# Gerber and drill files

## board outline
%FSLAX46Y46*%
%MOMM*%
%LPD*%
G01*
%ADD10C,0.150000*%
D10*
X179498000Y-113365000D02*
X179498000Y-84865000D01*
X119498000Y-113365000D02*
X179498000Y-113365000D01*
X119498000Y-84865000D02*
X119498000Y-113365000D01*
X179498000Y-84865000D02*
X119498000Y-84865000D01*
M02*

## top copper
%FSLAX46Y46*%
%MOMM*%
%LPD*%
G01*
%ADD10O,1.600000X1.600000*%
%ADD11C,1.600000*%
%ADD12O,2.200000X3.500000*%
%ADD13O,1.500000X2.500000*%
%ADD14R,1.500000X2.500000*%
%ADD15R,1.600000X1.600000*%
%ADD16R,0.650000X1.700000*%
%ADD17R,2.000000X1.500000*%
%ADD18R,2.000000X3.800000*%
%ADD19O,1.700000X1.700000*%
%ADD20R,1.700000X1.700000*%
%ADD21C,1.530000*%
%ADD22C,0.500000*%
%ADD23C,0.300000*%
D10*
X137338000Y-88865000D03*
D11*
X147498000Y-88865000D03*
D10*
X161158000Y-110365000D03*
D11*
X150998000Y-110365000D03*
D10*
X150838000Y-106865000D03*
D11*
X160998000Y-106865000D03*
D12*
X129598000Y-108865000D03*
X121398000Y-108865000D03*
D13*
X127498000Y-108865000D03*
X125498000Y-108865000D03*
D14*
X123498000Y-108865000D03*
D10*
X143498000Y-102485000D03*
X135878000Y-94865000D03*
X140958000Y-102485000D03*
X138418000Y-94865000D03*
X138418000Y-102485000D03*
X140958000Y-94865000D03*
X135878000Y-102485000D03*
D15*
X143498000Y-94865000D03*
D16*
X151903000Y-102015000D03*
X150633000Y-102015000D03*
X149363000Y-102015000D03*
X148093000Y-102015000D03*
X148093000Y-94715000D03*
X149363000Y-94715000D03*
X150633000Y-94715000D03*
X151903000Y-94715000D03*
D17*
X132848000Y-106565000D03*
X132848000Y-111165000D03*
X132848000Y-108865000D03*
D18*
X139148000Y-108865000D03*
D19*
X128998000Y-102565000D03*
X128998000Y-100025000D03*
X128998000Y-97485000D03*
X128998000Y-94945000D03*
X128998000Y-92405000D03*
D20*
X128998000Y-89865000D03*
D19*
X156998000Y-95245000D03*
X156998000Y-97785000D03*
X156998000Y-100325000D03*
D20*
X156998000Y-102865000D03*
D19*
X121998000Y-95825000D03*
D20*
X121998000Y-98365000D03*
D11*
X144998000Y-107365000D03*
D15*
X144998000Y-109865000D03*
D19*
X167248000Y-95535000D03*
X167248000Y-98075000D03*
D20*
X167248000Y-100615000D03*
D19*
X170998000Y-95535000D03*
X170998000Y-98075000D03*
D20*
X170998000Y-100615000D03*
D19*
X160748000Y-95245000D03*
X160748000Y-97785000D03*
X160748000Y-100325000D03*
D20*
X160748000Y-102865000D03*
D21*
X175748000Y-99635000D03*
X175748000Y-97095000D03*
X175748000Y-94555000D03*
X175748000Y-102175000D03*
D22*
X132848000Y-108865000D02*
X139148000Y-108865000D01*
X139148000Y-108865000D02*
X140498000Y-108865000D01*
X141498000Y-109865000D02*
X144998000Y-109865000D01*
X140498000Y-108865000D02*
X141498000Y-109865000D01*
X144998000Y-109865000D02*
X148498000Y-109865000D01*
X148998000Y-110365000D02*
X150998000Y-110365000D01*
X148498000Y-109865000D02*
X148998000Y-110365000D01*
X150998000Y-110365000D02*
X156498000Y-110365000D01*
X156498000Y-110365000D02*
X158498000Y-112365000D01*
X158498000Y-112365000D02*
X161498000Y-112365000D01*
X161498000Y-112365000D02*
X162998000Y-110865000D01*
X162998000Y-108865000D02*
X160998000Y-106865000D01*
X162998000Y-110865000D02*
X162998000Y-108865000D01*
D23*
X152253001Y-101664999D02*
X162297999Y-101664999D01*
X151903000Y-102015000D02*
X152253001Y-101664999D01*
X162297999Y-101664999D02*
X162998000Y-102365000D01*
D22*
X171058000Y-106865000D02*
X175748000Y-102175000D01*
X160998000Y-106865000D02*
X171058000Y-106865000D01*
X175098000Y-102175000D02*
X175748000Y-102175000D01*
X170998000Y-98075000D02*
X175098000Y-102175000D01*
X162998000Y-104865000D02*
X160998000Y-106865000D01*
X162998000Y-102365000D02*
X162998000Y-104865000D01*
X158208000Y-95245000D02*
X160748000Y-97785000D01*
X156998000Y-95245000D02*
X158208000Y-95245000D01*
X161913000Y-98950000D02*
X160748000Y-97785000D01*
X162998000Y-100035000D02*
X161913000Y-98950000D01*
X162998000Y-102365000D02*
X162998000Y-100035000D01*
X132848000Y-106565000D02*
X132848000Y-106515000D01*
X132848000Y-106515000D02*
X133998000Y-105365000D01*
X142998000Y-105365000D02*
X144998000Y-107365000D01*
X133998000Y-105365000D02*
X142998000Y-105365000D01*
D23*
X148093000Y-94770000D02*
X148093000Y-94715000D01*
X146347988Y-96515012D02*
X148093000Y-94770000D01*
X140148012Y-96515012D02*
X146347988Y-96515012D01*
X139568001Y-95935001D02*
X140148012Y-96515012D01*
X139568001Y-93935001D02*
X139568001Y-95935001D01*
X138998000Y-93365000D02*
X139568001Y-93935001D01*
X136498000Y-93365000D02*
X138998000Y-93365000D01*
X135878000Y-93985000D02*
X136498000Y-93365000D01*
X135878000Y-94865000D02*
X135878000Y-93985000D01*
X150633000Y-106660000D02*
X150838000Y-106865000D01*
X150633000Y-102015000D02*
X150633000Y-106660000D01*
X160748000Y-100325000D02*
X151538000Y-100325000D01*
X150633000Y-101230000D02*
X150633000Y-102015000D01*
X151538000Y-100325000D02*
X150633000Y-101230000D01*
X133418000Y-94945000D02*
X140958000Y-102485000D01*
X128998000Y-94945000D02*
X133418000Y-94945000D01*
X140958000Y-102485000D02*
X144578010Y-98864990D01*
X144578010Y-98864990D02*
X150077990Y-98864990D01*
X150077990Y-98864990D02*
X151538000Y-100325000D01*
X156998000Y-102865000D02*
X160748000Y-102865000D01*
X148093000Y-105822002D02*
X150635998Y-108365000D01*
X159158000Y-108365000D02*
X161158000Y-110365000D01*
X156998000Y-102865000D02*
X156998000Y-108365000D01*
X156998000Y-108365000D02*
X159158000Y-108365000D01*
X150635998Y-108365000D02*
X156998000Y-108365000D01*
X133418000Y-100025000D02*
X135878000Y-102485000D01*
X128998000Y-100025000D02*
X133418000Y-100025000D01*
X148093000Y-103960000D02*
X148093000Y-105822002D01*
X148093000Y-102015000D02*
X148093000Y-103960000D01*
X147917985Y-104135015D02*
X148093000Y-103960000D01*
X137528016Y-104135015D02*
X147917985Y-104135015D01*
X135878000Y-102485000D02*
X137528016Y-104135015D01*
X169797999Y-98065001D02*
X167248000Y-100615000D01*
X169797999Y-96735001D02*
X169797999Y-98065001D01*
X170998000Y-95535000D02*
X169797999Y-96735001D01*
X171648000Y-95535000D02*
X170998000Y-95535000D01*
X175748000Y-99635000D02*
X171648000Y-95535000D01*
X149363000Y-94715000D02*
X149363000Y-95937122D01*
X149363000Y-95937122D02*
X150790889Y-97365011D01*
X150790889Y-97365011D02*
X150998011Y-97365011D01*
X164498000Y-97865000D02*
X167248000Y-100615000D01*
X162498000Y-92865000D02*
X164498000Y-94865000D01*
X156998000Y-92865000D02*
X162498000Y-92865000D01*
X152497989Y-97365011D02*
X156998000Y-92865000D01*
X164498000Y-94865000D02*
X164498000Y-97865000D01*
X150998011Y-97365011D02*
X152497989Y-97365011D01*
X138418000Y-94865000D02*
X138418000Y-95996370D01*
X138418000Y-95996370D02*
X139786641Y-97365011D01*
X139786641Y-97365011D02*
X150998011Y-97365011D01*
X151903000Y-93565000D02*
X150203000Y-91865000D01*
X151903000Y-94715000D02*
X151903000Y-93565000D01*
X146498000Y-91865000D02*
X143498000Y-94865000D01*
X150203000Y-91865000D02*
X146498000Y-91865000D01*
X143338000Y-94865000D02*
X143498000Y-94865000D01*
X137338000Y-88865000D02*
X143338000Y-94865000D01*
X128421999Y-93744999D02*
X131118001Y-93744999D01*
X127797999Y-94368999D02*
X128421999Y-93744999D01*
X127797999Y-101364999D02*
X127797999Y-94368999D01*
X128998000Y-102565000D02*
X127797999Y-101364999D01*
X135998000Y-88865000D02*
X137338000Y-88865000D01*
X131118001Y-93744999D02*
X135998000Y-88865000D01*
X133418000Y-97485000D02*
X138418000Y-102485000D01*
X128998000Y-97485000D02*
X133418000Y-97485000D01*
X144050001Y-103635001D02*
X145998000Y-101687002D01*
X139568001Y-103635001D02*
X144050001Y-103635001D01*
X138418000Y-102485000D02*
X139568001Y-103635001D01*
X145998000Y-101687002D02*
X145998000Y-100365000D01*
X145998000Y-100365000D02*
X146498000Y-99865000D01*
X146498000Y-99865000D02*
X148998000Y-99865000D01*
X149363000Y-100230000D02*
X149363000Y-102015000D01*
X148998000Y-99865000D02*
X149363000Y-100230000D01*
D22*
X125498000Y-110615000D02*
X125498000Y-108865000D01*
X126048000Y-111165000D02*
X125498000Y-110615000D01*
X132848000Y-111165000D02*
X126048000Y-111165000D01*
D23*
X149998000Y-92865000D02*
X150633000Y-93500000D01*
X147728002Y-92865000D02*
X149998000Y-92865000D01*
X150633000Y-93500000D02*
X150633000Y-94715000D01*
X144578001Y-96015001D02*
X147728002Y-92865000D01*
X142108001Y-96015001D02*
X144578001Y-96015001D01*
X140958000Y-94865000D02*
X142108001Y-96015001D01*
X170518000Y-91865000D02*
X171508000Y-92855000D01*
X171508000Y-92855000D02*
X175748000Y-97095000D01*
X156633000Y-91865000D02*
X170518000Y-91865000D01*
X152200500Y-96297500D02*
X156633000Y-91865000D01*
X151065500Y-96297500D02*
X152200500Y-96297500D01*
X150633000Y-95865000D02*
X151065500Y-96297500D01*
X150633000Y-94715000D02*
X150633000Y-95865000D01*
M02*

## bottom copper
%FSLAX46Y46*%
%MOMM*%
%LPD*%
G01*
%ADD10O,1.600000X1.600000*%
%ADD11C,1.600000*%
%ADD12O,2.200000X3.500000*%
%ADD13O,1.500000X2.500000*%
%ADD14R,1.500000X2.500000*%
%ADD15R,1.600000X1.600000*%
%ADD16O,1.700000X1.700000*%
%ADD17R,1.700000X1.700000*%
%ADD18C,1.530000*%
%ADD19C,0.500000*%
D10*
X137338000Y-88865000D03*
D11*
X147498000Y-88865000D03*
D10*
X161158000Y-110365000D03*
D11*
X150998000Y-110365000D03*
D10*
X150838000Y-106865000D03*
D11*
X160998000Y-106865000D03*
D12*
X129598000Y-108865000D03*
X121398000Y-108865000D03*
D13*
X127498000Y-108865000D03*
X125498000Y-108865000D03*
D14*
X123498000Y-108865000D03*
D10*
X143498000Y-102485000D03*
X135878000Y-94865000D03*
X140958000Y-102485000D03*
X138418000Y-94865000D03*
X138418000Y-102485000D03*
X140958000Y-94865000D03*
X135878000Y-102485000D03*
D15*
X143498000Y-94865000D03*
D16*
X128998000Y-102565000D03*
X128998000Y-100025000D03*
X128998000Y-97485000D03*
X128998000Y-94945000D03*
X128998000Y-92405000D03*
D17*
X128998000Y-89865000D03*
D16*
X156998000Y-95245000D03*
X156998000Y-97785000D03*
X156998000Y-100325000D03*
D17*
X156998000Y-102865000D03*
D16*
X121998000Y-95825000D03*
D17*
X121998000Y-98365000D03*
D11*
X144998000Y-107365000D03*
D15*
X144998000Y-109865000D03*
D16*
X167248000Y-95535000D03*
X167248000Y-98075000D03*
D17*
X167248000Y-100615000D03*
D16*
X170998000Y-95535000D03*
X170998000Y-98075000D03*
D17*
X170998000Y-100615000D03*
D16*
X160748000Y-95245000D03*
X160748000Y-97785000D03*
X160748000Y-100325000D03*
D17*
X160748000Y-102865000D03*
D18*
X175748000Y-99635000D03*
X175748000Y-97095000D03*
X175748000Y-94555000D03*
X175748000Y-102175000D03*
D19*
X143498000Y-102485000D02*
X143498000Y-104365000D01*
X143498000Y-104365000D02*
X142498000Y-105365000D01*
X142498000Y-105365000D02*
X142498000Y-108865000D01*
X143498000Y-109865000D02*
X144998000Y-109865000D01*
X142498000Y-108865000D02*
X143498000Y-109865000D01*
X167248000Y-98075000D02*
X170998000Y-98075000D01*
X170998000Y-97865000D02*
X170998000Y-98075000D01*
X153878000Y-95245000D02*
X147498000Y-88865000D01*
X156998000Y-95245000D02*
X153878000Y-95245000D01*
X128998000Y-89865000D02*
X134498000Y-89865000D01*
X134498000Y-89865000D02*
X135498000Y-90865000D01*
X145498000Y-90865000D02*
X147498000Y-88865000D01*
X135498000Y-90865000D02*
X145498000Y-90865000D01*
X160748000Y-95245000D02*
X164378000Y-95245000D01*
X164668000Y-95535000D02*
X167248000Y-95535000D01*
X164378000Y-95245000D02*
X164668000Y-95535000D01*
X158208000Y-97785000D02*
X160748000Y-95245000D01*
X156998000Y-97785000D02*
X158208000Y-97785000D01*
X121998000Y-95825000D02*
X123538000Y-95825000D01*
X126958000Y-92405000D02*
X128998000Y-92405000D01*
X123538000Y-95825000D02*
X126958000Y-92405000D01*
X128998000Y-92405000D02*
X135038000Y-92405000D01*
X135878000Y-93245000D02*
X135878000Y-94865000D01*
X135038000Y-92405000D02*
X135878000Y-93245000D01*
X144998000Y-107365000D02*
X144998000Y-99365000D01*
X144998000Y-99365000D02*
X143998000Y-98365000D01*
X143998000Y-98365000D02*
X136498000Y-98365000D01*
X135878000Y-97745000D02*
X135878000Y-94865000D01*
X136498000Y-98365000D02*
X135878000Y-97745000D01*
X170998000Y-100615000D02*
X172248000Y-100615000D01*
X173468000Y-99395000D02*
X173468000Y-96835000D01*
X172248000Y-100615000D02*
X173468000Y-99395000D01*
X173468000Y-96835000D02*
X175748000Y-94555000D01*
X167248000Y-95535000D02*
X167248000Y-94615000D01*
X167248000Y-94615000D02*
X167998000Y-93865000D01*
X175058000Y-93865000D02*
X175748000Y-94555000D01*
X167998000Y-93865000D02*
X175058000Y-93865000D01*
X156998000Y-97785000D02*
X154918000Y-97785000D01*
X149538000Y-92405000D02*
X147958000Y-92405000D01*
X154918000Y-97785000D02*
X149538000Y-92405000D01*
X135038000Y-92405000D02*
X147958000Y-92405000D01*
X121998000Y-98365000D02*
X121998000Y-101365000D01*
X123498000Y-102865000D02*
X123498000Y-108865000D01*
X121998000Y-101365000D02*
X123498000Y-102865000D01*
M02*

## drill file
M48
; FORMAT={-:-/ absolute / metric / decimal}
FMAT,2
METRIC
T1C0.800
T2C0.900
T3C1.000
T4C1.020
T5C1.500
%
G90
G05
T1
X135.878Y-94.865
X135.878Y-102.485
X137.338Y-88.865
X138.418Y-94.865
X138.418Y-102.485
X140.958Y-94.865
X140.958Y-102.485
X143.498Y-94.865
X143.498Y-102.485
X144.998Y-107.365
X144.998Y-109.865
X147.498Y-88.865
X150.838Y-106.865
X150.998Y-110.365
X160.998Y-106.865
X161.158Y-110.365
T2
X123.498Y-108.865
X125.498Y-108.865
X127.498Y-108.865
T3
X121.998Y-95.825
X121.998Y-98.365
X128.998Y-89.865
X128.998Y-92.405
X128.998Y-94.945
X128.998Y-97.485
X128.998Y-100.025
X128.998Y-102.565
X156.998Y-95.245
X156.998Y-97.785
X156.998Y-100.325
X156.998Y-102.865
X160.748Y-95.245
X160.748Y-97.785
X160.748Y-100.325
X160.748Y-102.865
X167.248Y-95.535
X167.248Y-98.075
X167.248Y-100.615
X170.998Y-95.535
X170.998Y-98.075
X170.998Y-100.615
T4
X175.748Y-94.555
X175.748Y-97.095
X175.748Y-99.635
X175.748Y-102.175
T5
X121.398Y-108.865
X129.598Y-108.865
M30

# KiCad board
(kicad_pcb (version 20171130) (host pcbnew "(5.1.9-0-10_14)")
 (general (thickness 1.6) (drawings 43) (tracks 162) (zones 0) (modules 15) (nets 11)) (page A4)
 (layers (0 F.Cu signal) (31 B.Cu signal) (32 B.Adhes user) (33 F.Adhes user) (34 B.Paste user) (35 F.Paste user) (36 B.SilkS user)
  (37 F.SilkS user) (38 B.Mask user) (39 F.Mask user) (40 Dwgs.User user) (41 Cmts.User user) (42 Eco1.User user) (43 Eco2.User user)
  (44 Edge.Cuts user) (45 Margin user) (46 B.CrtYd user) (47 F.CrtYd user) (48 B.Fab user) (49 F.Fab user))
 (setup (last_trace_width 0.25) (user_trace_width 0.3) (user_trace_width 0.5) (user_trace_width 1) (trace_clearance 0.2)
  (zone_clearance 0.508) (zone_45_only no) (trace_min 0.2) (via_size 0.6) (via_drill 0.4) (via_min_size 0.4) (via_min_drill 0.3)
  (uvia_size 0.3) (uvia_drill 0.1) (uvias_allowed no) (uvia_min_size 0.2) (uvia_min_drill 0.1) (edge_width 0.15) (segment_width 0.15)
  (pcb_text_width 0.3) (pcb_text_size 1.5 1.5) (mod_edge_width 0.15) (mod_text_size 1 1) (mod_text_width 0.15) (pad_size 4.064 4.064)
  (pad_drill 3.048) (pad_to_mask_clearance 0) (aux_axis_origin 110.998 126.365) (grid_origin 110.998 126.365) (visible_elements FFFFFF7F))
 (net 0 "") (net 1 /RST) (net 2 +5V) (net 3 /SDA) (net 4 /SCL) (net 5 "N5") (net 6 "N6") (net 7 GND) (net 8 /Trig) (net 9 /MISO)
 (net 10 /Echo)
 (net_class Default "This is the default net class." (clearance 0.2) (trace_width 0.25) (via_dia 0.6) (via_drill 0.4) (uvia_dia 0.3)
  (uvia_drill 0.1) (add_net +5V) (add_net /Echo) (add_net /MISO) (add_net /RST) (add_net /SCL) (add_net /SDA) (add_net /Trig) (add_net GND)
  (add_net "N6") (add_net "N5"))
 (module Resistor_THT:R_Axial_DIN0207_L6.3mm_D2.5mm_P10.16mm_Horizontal (layer F.Cu) (at 147.498 88.865 180)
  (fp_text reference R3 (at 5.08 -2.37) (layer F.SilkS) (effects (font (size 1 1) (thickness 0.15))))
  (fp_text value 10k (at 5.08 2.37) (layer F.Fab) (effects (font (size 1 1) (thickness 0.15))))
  (pad 2 thru_hole oval (at 10.16 0 180) (size 1.6 1.6) (drill 0.8) (layers *.Cu *.Mask) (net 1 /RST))
  (pad 1 thru_hole circle (at 0 0 180) (size 1.6 1.6) (drill 0.8) (layers *.Cu *.Mask) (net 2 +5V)))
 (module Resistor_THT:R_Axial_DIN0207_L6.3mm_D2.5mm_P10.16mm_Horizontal (layer F.Cu) (at 150.998 110.365)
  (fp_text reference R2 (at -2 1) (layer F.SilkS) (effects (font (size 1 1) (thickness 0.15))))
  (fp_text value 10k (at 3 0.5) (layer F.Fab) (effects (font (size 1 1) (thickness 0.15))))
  (pad 2 thru_hole oval (at 10.16 0) (size 1.6 1.6) (drill 0.8) (layers *.Cu *.Mask) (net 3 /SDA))
  (pad 1 thru_hole circle (at 0 0) (size 1.6 1.6) (drill 0.8) (layers *.Cu *.Mask) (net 2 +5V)))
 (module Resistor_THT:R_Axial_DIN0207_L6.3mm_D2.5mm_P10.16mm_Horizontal (layer F.Cu) (at 160.998 106.865 180)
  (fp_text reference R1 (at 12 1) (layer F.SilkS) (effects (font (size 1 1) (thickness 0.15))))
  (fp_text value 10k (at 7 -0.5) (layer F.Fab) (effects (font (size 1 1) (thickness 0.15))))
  (pad 2 thru_hole oval (at 10.16 0 180) (size 1.6 1.6) (drill 0.8) (layers *.Cu *.Mask) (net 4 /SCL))
  (pad 1 thru_hole circle (at 0 0 180) (size 1.6 1.6) (drill 0.8) (layers *.Cu *.Mask) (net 2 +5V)))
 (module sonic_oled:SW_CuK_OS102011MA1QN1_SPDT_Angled (layer F.Cu) (at 123.498 108.865)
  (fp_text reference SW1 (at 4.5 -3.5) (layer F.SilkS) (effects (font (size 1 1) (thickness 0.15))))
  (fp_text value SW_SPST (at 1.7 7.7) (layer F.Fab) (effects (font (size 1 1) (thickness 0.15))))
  (pad "" thru_hole oval (at 6.1 0) (size 2.2 3.5) (drill 1.5) (layers *.Cu *.Mask))
  (pad "" thru_hole oval (at -2.1 0) (size 2.2 3.5) (drill 1.5) (layers *.Cu *.Mask))
  (pad 3 thru_hole oval (at 4 0) (size 1.5 2.5) (drill 0.9) (layers *.Cu *.Mask))
  (pad 2 thru_hole oval (at 2 0) (size 1.5 2.5) (drill 0.9) (layers *.Cu *.Mask) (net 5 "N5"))
  (pad 1 thru_hole rect (at 0 0) (size 1.5 2.5) (drill 0.9) (layers *.Cu *.Mask) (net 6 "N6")))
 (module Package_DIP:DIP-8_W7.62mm (layer F.Cu) (at 143.498 94.865 270)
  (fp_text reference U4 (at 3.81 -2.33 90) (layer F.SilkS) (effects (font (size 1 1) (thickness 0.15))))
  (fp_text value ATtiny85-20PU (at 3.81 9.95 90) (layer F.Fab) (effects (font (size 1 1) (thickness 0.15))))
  (pad 8 thru_hole oval (at 7.62 0 270) (size 1.6 1.6) (drill 0.8) (layers *.Cu *.Mask) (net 2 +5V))
  (pad 4 thru_hole oval (at 0 7.62 270) (size 1.6 1.6) (drill 0.8) (layers *.Cu *.Mask) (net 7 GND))
  (pad 7 thru_hole oval (at 7.62 2.54 270) (size 1.6 1.6) (drill 0.8) (layers *.Cu *.Mask) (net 4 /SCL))
  (pad 3 thru_hole oval (at 0 5.08 270) (size 1.6 1.6) (drill 0.8) (layers *.Cu *.Mask) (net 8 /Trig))
  (pad 6 thru_hole oval (at 7.62 5.08 270) (size 1.6 1.6) (drill 0.8) (layers *.Cu *.Mask) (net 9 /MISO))
  (pad 2 thru_hole oval (at 0 2.54 270) (size 1.6 1.6) (drill 0.8) (layers *.Cu *.Mask) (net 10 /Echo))
  (pad 5 thru_hole oval (at 7.62 7.62 270) (size 1.6 1.6) (drill 0.8) (layers *.Cu *.Mask) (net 3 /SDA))
  (pad 1 thru_hole rect (at 0 0 270) (size 1.6 1.6) (drill 0.8) (layers *.Cu *.Mask) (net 1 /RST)))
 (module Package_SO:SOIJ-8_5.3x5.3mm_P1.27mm (layer F.Cu) (at 149.998 98.365 270)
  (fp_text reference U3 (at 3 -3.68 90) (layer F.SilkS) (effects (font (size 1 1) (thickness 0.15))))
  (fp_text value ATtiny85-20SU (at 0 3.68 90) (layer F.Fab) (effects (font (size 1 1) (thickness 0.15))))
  (pad 8 smd rect (at 3.65 -1.905 270) (size 1.7 0.65) (layers F.Cu F.Paste F.Mask) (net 2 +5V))
  (pad 7 smd rect (at 3.65 -0.635 270) (size 1.7 0.65) (layers F.Cu F.Paste F.Mask) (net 4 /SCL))
  (pad 6 smd rect (at 3.65 0.635 270) (size 1.7 0.65) (layers F.Cu F.Paste F.Mask) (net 9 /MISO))
  (pad 5 smd rect (at 3.65 1.905 270) (size 1.7 0.65) (layers F.Cu F.Paste F.Mask) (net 3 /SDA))
  (pad 4 smd rect (at -3.65 1.905 270) (size 1.7 0.65) (layers F.Cu F.Paste F.Mask) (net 7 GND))
  (pad 3 smd rect (at -3.65 0.635 270) (size 1.7 0.65) (layers F.Cu F.Paste F.Mask) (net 8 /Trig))
  (pad 2 smd rect (at -3.65 -0.635 270) (size 1.7 0.65) (layers F.Cu F.Paste F.Mask) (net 10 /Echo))
  (pad 1 smd rect (at -3.65 -1.905 270) (size 1.7 0.65) (layers F.Cu F.Paste F.Mask) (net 1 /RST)))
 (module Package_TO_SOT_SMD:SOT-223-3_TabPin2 (layer F.Cu) (at 135.998 108.865)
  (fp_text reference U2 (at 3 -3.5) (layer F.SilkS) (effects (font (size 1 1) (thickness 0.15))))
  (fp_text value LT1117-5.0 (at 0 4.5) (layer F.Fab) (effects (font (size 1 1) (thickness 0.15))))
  (pad 1 smd rect (at -3.15 -2.3) (size 2 1.5) (layers F.Cu F.Paste F.Mask) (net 7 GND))
  (pad 3 smd rect (at -3.15 2.3) (size 2 1.5) (layers F.Cu F.Paste F.Mask) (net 5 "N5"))
  (pad 2 smd rect (at -3.15 0) (size 2 1.5) (layers F.Cu F.Paste F.Mask) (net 2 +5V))
  (pad 2 smd rect (at 3.15 0) (size 2 3.8) (layers F.Cu F.Paste F.Mask) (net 2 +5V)))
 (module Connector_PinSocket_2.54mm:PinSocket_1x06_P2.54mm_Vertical (layer F.Cu) (at 128.998 89.865)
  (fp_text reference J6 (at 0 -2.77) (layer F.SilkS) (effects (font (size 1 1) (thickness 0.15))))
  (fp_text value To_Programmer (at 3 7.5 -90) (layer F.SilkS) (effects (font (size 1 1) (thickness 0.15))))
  (pad 6 thru_hole oval (at 0 12.7) (size 1.7 1.7) (drill 1) (layers *.Cu *.Mask) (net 1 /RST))
  (pad 5 thru_hole oval (at 0 10.16) (size 1.7 1.7) (drill 1) (layers *.Cu *.Mask) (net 3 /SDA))
  (pad 4 thru_hole oval (at 0 7.62) (size 1.7 1.7) (drill 1) (layers *.Cu *.Mask) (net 9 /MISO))
  (pad 3 thru_hole oval (at 0 5.08) (size 1.7 1.7) (drill 1) (layers *.Cu *.Mask) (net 4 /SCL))
  (pad 2 thru_hole oval (at 0 2.54) (size 1.7 1.7) (drill 1) (layers *.Cu *.Mask) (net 7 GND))
  (pad 1 thru_hole rect (at 0 0) (size 1.7 1.7) (drill 1) (layers *.Cu *.Mask) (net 2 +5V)))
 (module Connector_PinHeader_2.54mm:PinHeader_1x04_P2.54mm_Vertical (layer F.Cu) (at 156.998 102.865 180)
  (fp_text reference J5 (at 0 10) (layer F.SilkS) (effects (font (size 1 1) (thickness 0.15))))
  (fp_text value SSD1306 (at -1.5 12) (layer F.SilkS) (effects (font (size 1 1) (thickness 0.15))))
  (pad 4 thru_hole oval (at 0 7.62 180) (size 1.7 1.7) (drill 1) (layers *.Cu *.Mask) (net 2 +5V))
  (pad 3 thru_hole oval (at 0 5.08 180) (size 1.7 1.7) (drill 1) (layers *.Cu *.Mask) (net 7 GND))
  (pad 2 thru_hole oval (at 0 2.54 180) (size 1.7 1.7) (drill 1) (layers *.Cu *.Mask) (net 4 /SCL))
  (pad 1 thru_hole rect (at 0 0 180) (size 1.7 1.7) (drill 1) (layers *.Cu *.Mask) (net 3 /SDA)))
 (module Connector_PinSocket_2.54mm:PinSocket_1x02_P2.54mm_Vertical (layer F.Cu) (at 121.998 98.365 180)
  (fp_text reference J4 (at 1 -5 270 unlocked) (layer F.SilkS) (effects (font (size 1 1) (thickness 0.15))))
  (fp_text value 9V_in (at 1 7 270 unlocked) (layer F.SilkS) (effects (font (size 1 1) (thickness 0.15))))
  (pad 2 thru_hole oval (at 0 2.54 180) (size 1.7 1.7) (drill 1) (layers *.Cu *.Mask) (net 7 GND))
  (pad 1 thru_hole rect (at 0 0 180) (size 1.7 1.7) (drill 1) (layers *.Cu *.Mask) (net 6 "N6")))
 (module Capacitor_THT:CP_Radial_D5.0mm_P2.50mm (layer F.Cu) (at 144.998 109.865 90)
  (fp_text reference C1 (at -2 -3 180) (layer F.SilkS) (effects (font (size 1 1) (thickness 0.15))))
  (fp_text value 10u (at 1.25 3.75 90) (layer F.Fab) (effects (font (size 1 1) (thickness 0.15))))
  (pad 2 thru_hole circle (at 2.5 0 90) (size 1.6 1.6) (drill 0.8) (layers *.Cu *.Mask) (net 7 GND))
  (pad 1 thru_hole rect (at 0 0 90) (size 1.6 1.6) (drill 0.8) (layers *.Cu *.Mask) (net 2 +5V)))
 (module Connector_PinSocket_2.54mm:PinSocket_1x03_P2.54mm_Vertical (layer F.Cu) (at 167.248 100.615 180)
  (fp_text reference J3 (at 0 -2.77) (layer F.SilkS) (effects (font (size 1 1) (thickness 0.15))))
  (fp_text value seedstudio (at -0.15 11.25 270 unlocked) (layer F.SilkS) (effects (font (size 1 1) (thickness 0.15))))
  (pad 3 thru_hole oval (at 0 5.08 180) (size 1.7 1.7) (drill 1) (layers *.Cu *.Mask) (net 7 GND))
  (pad 2 thru_hole oval (at 0 2.54 180) (size 1.7 1.7) (drill 1) (layers *.Cu *.Mask) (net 2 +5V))
  (pad 1 thru_hole rect (at 0 0 180) (size 1.7 1.7) (drill 1) (layers *.Cu *.Mask) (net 8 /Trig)))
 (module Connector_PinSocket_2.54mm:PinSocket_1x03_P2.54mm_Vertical (layer F.Cu) (at 170.998 100.615 180)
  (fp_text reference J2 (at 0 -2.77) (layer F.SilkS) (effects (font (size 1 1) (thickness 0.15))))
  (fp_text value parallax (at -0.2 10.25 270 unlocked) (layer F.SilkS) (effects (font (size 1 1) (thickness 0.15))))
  (pad 3 thru_hole oval (at 0 5.08 180) (size 1.7 1.7) (drill 1) (layers *.Cu *.Mask) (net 8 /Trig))
  (pad 2 thru_hole oval (at 0 2.54 180) (size 1.7 1.7) (drill 1) (layers *.Cu *.Mask) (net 2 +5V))
  (pad 1 thru_hole rect (at 0 0 180) (size 1.7 1.7) (drill 1) (layers *.Cu *.Mask) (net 7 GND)))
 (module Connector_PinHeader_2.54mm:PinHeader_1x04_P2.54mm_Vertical (layer F.Cu) (at 160.748 102.865 180)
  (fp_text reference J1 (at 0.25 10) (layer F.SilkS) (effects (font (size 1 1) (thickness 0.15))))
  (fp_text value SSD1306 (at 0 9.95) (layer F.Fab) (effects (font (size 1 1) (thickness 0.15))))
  (pad 4 thru_hole oval (at 0 7.62 180) (size 1.7 1.7) (drill 1) (layers *.Cu *.Mask) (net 7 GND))
  (pad 3 thru_hole oval (at 0 5.08 180) (size 1.7 1.7) (drill 1) (layers *.Cu *.Mask) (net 2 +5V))
  (pad 2 thru_hole oval (at 0 2.54 180) (size 1.7 1.7) (drill 1) (layers *.Cu *.Mask) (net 4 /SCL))
  (pad 1 thru_hole rect (at 0 0 180) (size 1.7 1.7) (drill 1) (layers *.Cu *.Mask) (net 3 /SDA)))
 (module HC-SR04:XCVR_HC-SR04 (layer F.Cu) (at 175.748 98.365 90)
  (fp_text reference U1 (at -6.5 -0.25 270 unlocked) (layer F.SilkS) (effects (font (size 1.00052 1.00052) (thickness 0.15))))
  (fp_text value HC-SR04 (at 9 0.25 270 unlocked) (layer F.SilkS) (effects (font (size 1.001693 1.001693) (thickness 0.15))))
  (pad 2 thru_hole circle (at -1.27 0 90) (size 1.53 1.53) (drill 1.02) (layers *.Cu *.Mask) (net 8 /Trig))
  (pad 3 thru_hole circle (at 1.27 0 90) (size 1.53 1.53) (drill 1.02) (layers *.Cu *.Mask) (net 10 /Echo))
  (pad 4 thru_hole circle (at 3.81 0 90) (size 1.53 1.53) (drill 1.02) (layers *.Cu *.Mask) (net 7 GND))
  (pad 1 thru_hole circle (at -3.81 0 90) (size 1.53 1.53) (drill 1.02) (layers *.Cu *.Mask) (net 2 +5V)))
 (gr_line (start 179.498 113.365) (end 179.498 84.865) (angle 90) (layer Edge.Cuts) (width 0.15))
 (gr_line (start 119.498 113.365) (end 179.498 113.365) (angle 90) (layer Edge.Cuts) (width 0.15))
 (gr_line (start 119.498 84.865) (end 119.498 113.365) (angle 90) (layer Edge.Cuts) (width 0.15))
 (gr_line (start 179.498 84.865) (end 119.498 84.865) (angle 90) (layer Edge.Cuts) (width 0.15))
 (segment (start 132.848 108.865) (end 139.148 108.865) (width 0.5) (layer F.Cu) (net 2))
 (segment (start 139.148 108.865) (end 140.498 108.865) (width 0.5) (layer F.Cu) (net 2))
 (segment (start 141.498 109.865) (end 144.998 109.865) (width 0.5) (layer F.Cu) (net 2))
 (segment (start 140.498 108.865) (end 141.498 109.865) (width 0.5) (layer F.Cu) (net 2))
 (segment (start 144.998 109.865) (end 148.498 109.865) (width 0.5) (layer F.Cu) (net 2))
 (segment (start 148.998 110.365) (end 150.998 110.365) (width 0.5) (layer F.Cu) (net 2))
 (segment (start 148.498 109.865) (end 148.998 110.365) (width 0.5) (layer F.Cu) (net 2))
 (segment (start 150.998 110.365) (end 156.498 110.365) (width 0.5) (layer F.Cu) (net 2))
 (segment (start 156.498 110.365) (end 158.498 112.365) (width 0.5) (layer F.Cu) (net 2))
 (segment (start 158.498 112.365) (end 161.498 112.365) (width 0.5) (layer F.Cu) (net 2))
 (segment (start 161.498 112.365) (end 162.998 110.865) (width 0.5) (layer F.Cu) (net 2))
 (segment (start 162.998 108.865) (end 160.998 106.865) (width 0.5) (layer F.Cu) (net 2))
 (segment (start 162.998 110.865) (end 162.998 108.865) (width 0.5) (layer F.Cu) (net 2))
 (segment (start 143.498 102.485) (end 143.498 104.365) (width 0.5) (layer B.Cu) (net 2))
 (segment (start 143.498 104.365) (end 142.498 105.365) (width 0.5) (layer B.Cu) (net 2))
 (segment (start 142.498 105.365) (end 142.498 108.865) (width 0.5) (layer B.Cu) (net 2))
 (segment (start 143.498 109.865) (end 144.998 109.865) (width 0.5) (layer B.Cu) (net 2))
 (segment (start 142.498 108.865) (end 143.498 109.865) (width 0.5) (layer B.Cu) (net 2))
 (segment (start 152.253001 101.664999) (end 162.297999 101.664999) (width 0.3) (layer F.Cu) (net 2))
 (segment (start 151.903 102.015) (end 152.253001 101.664999) (width 0.3) (layer F.Cu) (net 2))
 (segment (start 162.297999 101.664999) (end 162.998 102.365) (width 0.3) (layer F.Cu) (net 2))
 (segment (start 171.058 106.865) (end 175.748 102.175) (width 0.5) (layer F.Cu) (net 2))
 (segment (start 160.998 106.865) (end 171.058 106.865) (width 0.5) (layer F.Cu) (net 2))
 (segment (start 167.248 98.075) (end 170.998 98.075) (width 0.5) (layer B.Cu) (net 2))
 (segment (start 170.998 97.865) (end 170.998 98.075) (width 0.5) (layer B.Cu) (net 2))
 (segment (start 175.098 102.175) (end 175.748 102.175) (width 0.5) (layer F.Cu) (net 2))
 (segment (start 170.998 98.075) (end 175.098 102.175) (width 0.5) (layer F.Cu) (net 2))
 (segment (start 162.998 104.865) (end 160.998 106.865) (width 0.5) (layer F.Cu) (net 2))
 (segment (start 162.998 102.365) (end 162.998 104.865) (width 0.5) (layer F.Cu) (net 2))
 (segment (start 158.208 95.245) (end 160.748 97.785) (width 0.5) (layer F.Cu) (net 2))
 (segment (start 156.998 95.245) (end 158.208 95.245) (width 0.5) (layer F.Cu) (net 2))
 (segment (start 161.913 98.95) (end 160.748 97.785) (width 0.5) (layer F.Cu) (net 2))
 (segment (start 162.998 100.035) (end 161.913 98.95) (width 0.5) (layer F.Cu) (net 2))
 (segment (start 162.998 102.365) (end 162.998 100.035) (width 0.5) (layer F.Cu) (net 2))
 (segment (start 153.878 95.245) (end 147.498 88.865) (width 0.5) (layer B.Cu) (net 2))
 (segment (start 156.998 95.245) (end 153.878 95.245) (width 0.5) (layer B.Cu) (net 2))
 (segment (start 128.998 89.865) (end 134.498 89.865) (width 0.5) (layer B.Cu) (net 2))
 (segment (start 134.498 89.865) (end 135.498 90.865) (width 0.5) (layer B.Cu) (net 2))
 (segment (start 145.498 90.865) (end 147.498 88.865) (width 0.5) (layer B.Cu) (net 2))
 (segment (start 135.498 90.865) (end 145.498 90.865) (width 0.5) (layer B.Cu) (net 2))
 (segment (start 160.748 95.245) (end 164.378 95.245) (width 0.5) (layer B.Cu) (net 7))
 (segment (start 164.668 95.535) (end 167.248 95.535) (width 0.5) (layer B.Cu) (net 7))
 (segment (start 164.378 95.245) (end 164.668 95.535) (width 0.5) (layer B.Cu) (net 7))
 (segment (start 158.208 97.785) (end 160.748 95.245) (width 0.5) (layer B.Cu) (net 7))
 (segment (start 156.998 97.785) (end 158.208 97.785) (width 0.5) (layer B.Cu) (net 7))
 (segment (start 121.998 95.825) (end 123.538 95.825) (width 0.5) (layer B.Cu) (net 7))
 (segment (start 126.958 92.405) (end 128.998 92.405) (width 0.5) (layer B.Cu) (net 7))
 (segment (start 123.538 95.825) (end 126.958 92.405) (width 0.5) (layer B.Cu) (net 7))
 (segment (start 128.998 92.405) (end 135.038 92.405) (width 0.5) (layer B.Cu) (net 7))
 (segment (start 135.878 93.245) (end 135.878 94.865) (width 0.5) (layer B.Cu) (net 7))
 (segment (start 135.038 92.405) (end 135.878 93.245) (width 0.5) (layer B.Cu) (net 7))
 (segment (start 132.848 106.565) (end 132.848 106.515) (width 0.5) (layer F.Cu) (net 7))
 (segment (start 132.848 106.515) (end 133.998 105.365) (width 0.5) (layer F.Cu) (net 7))
 (segment (start 142.998 105.365) (end 144.998 107.365) (width 0.5) (layer F.Cu) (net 7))
 (segment (start 133.998 105.365) (end 142.998 105.365) (width 0.5) (layer F.Cu) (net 7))
 (segment (start 148.093 94.77) (end 148.093 94.715) (width 0.3) (layer F.Cu) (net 7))
 (segment (start 146.347988 96.515012) (end 148.093 94.77) (width 0.3) (layer F.Cu) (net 7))
 (segment (start 140.148012 96.515012) (end 146.347988 96.515012) (width 0.3) (layer F.Cu) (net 7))
 (segment (start 139.568001 95.935001) (end 140.148012 96.515012) (width 0.3) (layer F.Cu) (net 7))
 (segment (start 139.568001 93.935001) (end 139.568001 95.935001) (width 0.3) (layer F.Cu) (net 7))
 (segment (start 138.998 93.365) (end 139.568001 93.935001) (width 0.3) (layer F.Cu) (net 7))
 (segment (start 136.498 93.365) (end 138.998 93.365) (width 0.3) (layer F.Cu) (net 7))
 (segment (start 135.878 93.985) (end 136.498 93.365) (width 0.3) (layer F.Cu) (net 7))
 (segment (start 135.878 94.865) (end 135.878 93.985) (width 0.3) (layer F.Cu) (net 7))
 (segment (start 144.998 107.365) (end 144.998 99.365) (width 0.5) (layer B.Cu) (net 7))
 (segment (start 144.998 99.365) (end 143.998 98.365) (width 0.5) (layer B.Cu) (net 7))
 (segment (start 143.998 98.365) (end 136.498 98.365) (width 0.5) (layer B.Cu) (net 7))
 (segment (start 135.878 97.745) (end 135.878 94.865) (width 0.5) (layer B.Cu) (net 7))
 (segment (start 136.498 98.365) (end 135.878 97.745) (width 0.5) (layer B.Cu) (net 7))
 (segment (start 170.998 100.615) (end 172.248 100.615) (width 0.5) (layer B.Cu) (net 7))
 (segment (start 173.468 99.395) (end 173.468 96.835) (width 0.5) (layer B.Cu) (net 7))
 (segment (start 172.248 100.615) (end 173.468 99.395) (width 0.5) (layer B.Cu) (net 7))
 (segment (start 173.468 96.835) (end 175.748 94.555) (width 0.5) (layer B.Cu) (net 7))
 (segment (start 167.248 95.535) (end 167.248 94.615) (width 0.5) (layer B.Cu) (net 7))
 (segment (start 167.248 94.615) (end 167.998 93.865) (width 0.5) (layer B.Cu) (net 7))
 (segment (start 175.058 93.865) (end 175.748 94.555) (width 0.5) (layer B.Cu) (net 7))
 (segment (start 167.998 93.865) (end 175.058 93.865) (width 0.5) (layer B.Cu) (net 7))
 (segment (start 156.998 97.785) (end 154.918 97.785) (width 0.5) (layer B.Cu) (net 7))
 (segment (start 149.538 92.405) (end 147.958 92.405) (width 0.5) (layer B.Cu) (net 7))
 (segment (start 154.918 97.785) (end 149.538 92.405) (width 0.5) (layer B.Cu) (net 7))
 (segment (start 135.038 92.405) (end 147.958 92.405) (width 0.5) (layer B.Cu) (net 7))
 (segment (start 150.633 106.66) (end 150.838 106.865) (width 0.3) (layer F.Cu) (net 4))
 (segment (start 150.633 102.015) (end 150.633 106.66) (width 0.3) (layer F.Cu) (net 4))
 (segment (start 160.748 100.325) (end 151.538 100.325) (width 0.3) (layer F.Cu) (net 4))
 (segment (start 150.633 101.23) (end 150.633 102.015) (width 0.3) (layer F.Cu) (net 4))
 (segment (start 151.538 100.325) (end 150.633 101.23) (width 0.3) (layer F.Cu) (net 4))
 (segment (start 133.418 94.945) (end 140.958 102.485) (width 0.3) (layer F.Cu) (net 4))
 (segment (start 128.998 94.945) (end 133.418 94.945) (width 0.3) (layer F.Cu) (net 4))
 (segment (start 140.958 102.485) (end 144.57801 98.86499) (width 0.3) (layer F.Cu) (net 4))
 (segment (start 144.57801 98.86499) (end 150.07799 98.86499) (width 0.3) (layer F.Cu) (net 4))
 (segment (start 150.07799 98.86499) (end 151.538 100.325) (width 0.3) (layer F.Cu) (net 4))
 (segment (start 156.998 102.865) (end 160.748 102.865) (width 0.3) (layer F.Cu) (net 3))
 (segment (start 148.093 105.822002) (end 150.635998 108.365) (width 0.3) (layer F.Cu) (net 3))
 (segment (start 159.158 108.365) (end 161.158 110.365) (width 0.3) (layer F.Cu) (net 3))
 (segment (start 156.998 102.865) (end 156.998 108.365) (width 0.3) (layer F.Cu) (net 3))
 (segment (start 156.998 108.365) (end 159.158 108.365) (width 0.3) (layer F.Cu) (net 3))
 (segment (start 150.635998 108.365) (end 156.998 108.365) (width 0.3) (layer F.Cu) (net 3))
 (segment (start 133.418 100.025) (end 135.878 102.485) (width 0.3) (layer F.Cu) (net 3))
 (segment (start 128.998 100.025) (end 133.418 100.025) (width 0.3) (layer F.Cu) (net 3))
 (segment (start 148.093 103.96) (end 148.093 105.822002) (width 0.3) (layer F.Cu) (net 3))
 (segment (start 148.093 102.015) (end 148.093 103.96) (width 0.3) (layer F.Cu) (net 3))
 (segment (start 147.917985 104.135015) (end 148.093 103.96) (width 0.3) (layer F.Cu) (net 3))
 (segment (start 137.528016 104.135015) (end 147.917985 104.135015) (width 0.3) (layer F.Cu) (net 3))
 (segment (start 135.878 102.485) (end 137.528016 104.135015) (width 0.3) (layer F.Cu) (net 3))
 (segment (start 169.797999 98.065001) (end 167.248 100.615) (width 0.3) (layer F.Cu) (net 8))
 (segment (start 169.797999 96.735001) (end 169.797999 98.065001) (width 0.3) (layer F.Cu) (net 8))
 (segment (start 170.998 95.535) (end 169.797999 96.735001) (width 0.3) (layer F.Cu) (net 8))
 (segment (start 171.648 95.535) (end 170.998 95.535) (width 0.3) (layer F.Cu) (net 8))
 (segment (start 175.748 99.635) (end 171.648 95.535) (width 0.3) (layer F.Cu) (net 8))
 (segment (start 149.363 94.715) (end 149.363 95.937122) (width 0.3) (layer F.Cu) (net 8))
 (segment (start 149.363 95.937122) (end 150.790889 97.365011) (width 0.3) (layer F.Cu) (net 8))
 (segment (start 150.790889 97.365011) (end 150.998011 97.365011) (width 0.3) (layer F.Cu) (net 8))
 (segment (start 164.498 97.865) (end 167.248 100.615) (width 0.3) (layer F.Cu) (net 8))
 (segment (start 162.498 92.865) (end 164.498 94.865) (width 0.3) (layer F.Cu) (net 8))
 (segment (start 156.998 92.865) (end 162.498 92.865) (width 0.3) (layer F.Cu) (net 8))
 (segment (start 152.497989 97.365011) (end 156.998 92.865) (width 0.3) (layer F.Cu) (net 8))
 (segment (start 164.498 94.865) (end 164.498 97.865) (width 0.3) (layer F.Cu) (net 8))
 (segment (start 150.998011 97.365011) (end 152.497989 97.365011) (width 0.3) (layer F.Cu) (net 8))
 (segment (start 138.418 94.865) (end 138.418 95.99637) (width 0.3) (layer F.Cu) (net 8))
 (segment (start 138.418 95.99637) (end 139.786641 97.365011) (width 0.3) (layer F.Cu) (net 8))
 (segment (start 139.786641 97.365011) (end 150.998011 97.365011) (width 0.3) (layer F.Cu) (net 8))
 (segment (start 121.998 98.365) (end 121.998 101.365) (width 0.5) (layer B.Cu) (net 6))
 (segment (start 123.498 102.865) (end 123.498 108.865) (width 0.5) (layer B.Cu) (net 6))
 (segment (start 121.998 101.365) (end 123.498 102.865) (width 0.5) (layer B.Cu) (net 6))
 (segment (start 151.903 93.565) (end 150.203 91.865) (width 0.3) (layer F.Cu) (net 1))
 (segment (start 151.903 94.715) (end 151.903 93.565) (width 0.3) (layer F.Cu) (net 1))
 (segment (start 146.498 91.865) (end 143.498 94.865) (width 0.3) (layer F.Cu) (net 1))
 (segment (start 150.203 91.865) (end 146.498 91.865) (width 0.3) (layer F.Cu) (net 1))
 (segment (start 143.338 94.865) (end 143.498 94.865) (width 0.3) (layer F.Cu) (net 1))
 (segment (start 137.338 88.865) (end 143.338 94.865) (width 0.3) (layer F.Cu) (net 1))
 (segment (start 128.421999 93.744999) (end 131.118001 93.744999) (width 0.3) (layer F.Cu) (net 1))
 (segment (start 127.797999 94.368999) (end 128.421999 93.744999) (width 0.3) (layer F.Cu) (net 1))
 (segment (start 127.797999 101.364999) (end 127.797999 94.368999) (width 0.3) (layer F.Cu) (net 1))
 (segment (start 128.998 102.565) (end 127.797999 101.364999) (width 0.3) (layer F.Cu) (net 1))
 (segment (start 135.998 88.865) (end 137.338 88.865) (width 0.3) (layer F.Cu) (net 1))
 (segment (start 131.118001 93.744999) (end 135.998 88.865) (width 0.3) (layer F.Cu) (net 1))
 (segment (start 133.418 97.485) (end 138.418 102.485) (width 0.3) (layer F.Cu) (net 9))
 (segment (start 128.998 97.485) (end 133.418 97.485) (width 0.3) (layer F.Cu) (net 9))
 (segment (start 144.050001 103.635001) (end 145.998 101.687002) (width 0.3) (layer F.Cu) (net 9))
 (segment (start 139.568001 103.635001) (end 144.050001 103.635001) (width 0.3) (layer F.Cu) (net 9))
 (segment (start 138.418 102.485) (end 139.568001 103.635001) (width 0.3) (layer F.Cu) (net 9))
 (segment (start 145.998 101.687002) (end 145.998 100.365) (width 0.3) (layer F.Cu) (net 9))
 (segment (start 145.998 100.365) (end 146.498 99.865) (width 0.3) (layer F.Cu) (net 9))
 (segment (start 146.498 99.865) (end 148.998 99.865) (width 0.3) (layer F.Cu) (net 9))
 (segment (start 149.363 100.23) (end 149.363 102.015) (width 0.3) (layer F.Cu) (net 9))
 (segment (start 148.998 99.865) (end 149.363 100.23) (width 0.3) (layer F.Cu) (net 9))
 (segment (start 125.498 110.615) (end 125.498 108.865) (width 0.5) (layer F.Cu) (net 5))
 (segment (start 126.048 111.165) (end 125.498 110.615) (width 0.5) (layer F.Cu) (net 5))
 (segment (start 132.848 111.165) (end 126.048 111.165) (width 0.5) (layer F.Cu) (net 5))
 (segment (start 149.998 92.865) (end 150.633 93.5) (width 0.3) (layer F.Cu) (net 10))
 (segment (start 147.728002 92.865) (end 149.998 92.865) (width 0.3) (layer F.Cu) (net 10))
 (segment (start 150.633 93.5) (end 150.633 94.715) (width 0.3) (layer F.Cu) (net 10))
 (segment (start 144.578001 96.015001) (end 147.728002 92.865) (width 0.3) (layer F.Cu) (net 10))
 (segment (start 142.108001 96.015001) (end 144.578001 96.015001) (width 0.3) (layer F.Cu) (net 10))
 (segment (start 140.958 94.865) (end 142.108001 96.015001) (width 0.3) (layer F.Cu) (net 10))
 (segment (start 170.518 91.865) (end 171.508 92.855) (width 0.3) (layer F.Cu) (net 10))
 (segment (start 171.508 92.855) (end 175.748 97.095) (width 0.3) (layer F.Cu) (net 10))
 (segment (start 156.633 91.865) (end 170.518 91.865) (width 0.3) (layer F.Cu) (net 10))
 (segment (start 152.2005 96.2975) (end 156.633 91.865) (width 0.3) (layer F.Cu) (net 10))
 (segment (start 151.0655 96.2975) (end 152.2005 96.2975) (width 0.3) (layer F.Cu) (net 10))
 (segment (start 150.633 95.865) (end 151.0655 96.2975) (width 0.3) (layer F.Cu) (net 10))
 (segment (start 150.633 94.715) (end 150.633 95.865) (width 0.3) (layer F.Cu) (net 10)))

